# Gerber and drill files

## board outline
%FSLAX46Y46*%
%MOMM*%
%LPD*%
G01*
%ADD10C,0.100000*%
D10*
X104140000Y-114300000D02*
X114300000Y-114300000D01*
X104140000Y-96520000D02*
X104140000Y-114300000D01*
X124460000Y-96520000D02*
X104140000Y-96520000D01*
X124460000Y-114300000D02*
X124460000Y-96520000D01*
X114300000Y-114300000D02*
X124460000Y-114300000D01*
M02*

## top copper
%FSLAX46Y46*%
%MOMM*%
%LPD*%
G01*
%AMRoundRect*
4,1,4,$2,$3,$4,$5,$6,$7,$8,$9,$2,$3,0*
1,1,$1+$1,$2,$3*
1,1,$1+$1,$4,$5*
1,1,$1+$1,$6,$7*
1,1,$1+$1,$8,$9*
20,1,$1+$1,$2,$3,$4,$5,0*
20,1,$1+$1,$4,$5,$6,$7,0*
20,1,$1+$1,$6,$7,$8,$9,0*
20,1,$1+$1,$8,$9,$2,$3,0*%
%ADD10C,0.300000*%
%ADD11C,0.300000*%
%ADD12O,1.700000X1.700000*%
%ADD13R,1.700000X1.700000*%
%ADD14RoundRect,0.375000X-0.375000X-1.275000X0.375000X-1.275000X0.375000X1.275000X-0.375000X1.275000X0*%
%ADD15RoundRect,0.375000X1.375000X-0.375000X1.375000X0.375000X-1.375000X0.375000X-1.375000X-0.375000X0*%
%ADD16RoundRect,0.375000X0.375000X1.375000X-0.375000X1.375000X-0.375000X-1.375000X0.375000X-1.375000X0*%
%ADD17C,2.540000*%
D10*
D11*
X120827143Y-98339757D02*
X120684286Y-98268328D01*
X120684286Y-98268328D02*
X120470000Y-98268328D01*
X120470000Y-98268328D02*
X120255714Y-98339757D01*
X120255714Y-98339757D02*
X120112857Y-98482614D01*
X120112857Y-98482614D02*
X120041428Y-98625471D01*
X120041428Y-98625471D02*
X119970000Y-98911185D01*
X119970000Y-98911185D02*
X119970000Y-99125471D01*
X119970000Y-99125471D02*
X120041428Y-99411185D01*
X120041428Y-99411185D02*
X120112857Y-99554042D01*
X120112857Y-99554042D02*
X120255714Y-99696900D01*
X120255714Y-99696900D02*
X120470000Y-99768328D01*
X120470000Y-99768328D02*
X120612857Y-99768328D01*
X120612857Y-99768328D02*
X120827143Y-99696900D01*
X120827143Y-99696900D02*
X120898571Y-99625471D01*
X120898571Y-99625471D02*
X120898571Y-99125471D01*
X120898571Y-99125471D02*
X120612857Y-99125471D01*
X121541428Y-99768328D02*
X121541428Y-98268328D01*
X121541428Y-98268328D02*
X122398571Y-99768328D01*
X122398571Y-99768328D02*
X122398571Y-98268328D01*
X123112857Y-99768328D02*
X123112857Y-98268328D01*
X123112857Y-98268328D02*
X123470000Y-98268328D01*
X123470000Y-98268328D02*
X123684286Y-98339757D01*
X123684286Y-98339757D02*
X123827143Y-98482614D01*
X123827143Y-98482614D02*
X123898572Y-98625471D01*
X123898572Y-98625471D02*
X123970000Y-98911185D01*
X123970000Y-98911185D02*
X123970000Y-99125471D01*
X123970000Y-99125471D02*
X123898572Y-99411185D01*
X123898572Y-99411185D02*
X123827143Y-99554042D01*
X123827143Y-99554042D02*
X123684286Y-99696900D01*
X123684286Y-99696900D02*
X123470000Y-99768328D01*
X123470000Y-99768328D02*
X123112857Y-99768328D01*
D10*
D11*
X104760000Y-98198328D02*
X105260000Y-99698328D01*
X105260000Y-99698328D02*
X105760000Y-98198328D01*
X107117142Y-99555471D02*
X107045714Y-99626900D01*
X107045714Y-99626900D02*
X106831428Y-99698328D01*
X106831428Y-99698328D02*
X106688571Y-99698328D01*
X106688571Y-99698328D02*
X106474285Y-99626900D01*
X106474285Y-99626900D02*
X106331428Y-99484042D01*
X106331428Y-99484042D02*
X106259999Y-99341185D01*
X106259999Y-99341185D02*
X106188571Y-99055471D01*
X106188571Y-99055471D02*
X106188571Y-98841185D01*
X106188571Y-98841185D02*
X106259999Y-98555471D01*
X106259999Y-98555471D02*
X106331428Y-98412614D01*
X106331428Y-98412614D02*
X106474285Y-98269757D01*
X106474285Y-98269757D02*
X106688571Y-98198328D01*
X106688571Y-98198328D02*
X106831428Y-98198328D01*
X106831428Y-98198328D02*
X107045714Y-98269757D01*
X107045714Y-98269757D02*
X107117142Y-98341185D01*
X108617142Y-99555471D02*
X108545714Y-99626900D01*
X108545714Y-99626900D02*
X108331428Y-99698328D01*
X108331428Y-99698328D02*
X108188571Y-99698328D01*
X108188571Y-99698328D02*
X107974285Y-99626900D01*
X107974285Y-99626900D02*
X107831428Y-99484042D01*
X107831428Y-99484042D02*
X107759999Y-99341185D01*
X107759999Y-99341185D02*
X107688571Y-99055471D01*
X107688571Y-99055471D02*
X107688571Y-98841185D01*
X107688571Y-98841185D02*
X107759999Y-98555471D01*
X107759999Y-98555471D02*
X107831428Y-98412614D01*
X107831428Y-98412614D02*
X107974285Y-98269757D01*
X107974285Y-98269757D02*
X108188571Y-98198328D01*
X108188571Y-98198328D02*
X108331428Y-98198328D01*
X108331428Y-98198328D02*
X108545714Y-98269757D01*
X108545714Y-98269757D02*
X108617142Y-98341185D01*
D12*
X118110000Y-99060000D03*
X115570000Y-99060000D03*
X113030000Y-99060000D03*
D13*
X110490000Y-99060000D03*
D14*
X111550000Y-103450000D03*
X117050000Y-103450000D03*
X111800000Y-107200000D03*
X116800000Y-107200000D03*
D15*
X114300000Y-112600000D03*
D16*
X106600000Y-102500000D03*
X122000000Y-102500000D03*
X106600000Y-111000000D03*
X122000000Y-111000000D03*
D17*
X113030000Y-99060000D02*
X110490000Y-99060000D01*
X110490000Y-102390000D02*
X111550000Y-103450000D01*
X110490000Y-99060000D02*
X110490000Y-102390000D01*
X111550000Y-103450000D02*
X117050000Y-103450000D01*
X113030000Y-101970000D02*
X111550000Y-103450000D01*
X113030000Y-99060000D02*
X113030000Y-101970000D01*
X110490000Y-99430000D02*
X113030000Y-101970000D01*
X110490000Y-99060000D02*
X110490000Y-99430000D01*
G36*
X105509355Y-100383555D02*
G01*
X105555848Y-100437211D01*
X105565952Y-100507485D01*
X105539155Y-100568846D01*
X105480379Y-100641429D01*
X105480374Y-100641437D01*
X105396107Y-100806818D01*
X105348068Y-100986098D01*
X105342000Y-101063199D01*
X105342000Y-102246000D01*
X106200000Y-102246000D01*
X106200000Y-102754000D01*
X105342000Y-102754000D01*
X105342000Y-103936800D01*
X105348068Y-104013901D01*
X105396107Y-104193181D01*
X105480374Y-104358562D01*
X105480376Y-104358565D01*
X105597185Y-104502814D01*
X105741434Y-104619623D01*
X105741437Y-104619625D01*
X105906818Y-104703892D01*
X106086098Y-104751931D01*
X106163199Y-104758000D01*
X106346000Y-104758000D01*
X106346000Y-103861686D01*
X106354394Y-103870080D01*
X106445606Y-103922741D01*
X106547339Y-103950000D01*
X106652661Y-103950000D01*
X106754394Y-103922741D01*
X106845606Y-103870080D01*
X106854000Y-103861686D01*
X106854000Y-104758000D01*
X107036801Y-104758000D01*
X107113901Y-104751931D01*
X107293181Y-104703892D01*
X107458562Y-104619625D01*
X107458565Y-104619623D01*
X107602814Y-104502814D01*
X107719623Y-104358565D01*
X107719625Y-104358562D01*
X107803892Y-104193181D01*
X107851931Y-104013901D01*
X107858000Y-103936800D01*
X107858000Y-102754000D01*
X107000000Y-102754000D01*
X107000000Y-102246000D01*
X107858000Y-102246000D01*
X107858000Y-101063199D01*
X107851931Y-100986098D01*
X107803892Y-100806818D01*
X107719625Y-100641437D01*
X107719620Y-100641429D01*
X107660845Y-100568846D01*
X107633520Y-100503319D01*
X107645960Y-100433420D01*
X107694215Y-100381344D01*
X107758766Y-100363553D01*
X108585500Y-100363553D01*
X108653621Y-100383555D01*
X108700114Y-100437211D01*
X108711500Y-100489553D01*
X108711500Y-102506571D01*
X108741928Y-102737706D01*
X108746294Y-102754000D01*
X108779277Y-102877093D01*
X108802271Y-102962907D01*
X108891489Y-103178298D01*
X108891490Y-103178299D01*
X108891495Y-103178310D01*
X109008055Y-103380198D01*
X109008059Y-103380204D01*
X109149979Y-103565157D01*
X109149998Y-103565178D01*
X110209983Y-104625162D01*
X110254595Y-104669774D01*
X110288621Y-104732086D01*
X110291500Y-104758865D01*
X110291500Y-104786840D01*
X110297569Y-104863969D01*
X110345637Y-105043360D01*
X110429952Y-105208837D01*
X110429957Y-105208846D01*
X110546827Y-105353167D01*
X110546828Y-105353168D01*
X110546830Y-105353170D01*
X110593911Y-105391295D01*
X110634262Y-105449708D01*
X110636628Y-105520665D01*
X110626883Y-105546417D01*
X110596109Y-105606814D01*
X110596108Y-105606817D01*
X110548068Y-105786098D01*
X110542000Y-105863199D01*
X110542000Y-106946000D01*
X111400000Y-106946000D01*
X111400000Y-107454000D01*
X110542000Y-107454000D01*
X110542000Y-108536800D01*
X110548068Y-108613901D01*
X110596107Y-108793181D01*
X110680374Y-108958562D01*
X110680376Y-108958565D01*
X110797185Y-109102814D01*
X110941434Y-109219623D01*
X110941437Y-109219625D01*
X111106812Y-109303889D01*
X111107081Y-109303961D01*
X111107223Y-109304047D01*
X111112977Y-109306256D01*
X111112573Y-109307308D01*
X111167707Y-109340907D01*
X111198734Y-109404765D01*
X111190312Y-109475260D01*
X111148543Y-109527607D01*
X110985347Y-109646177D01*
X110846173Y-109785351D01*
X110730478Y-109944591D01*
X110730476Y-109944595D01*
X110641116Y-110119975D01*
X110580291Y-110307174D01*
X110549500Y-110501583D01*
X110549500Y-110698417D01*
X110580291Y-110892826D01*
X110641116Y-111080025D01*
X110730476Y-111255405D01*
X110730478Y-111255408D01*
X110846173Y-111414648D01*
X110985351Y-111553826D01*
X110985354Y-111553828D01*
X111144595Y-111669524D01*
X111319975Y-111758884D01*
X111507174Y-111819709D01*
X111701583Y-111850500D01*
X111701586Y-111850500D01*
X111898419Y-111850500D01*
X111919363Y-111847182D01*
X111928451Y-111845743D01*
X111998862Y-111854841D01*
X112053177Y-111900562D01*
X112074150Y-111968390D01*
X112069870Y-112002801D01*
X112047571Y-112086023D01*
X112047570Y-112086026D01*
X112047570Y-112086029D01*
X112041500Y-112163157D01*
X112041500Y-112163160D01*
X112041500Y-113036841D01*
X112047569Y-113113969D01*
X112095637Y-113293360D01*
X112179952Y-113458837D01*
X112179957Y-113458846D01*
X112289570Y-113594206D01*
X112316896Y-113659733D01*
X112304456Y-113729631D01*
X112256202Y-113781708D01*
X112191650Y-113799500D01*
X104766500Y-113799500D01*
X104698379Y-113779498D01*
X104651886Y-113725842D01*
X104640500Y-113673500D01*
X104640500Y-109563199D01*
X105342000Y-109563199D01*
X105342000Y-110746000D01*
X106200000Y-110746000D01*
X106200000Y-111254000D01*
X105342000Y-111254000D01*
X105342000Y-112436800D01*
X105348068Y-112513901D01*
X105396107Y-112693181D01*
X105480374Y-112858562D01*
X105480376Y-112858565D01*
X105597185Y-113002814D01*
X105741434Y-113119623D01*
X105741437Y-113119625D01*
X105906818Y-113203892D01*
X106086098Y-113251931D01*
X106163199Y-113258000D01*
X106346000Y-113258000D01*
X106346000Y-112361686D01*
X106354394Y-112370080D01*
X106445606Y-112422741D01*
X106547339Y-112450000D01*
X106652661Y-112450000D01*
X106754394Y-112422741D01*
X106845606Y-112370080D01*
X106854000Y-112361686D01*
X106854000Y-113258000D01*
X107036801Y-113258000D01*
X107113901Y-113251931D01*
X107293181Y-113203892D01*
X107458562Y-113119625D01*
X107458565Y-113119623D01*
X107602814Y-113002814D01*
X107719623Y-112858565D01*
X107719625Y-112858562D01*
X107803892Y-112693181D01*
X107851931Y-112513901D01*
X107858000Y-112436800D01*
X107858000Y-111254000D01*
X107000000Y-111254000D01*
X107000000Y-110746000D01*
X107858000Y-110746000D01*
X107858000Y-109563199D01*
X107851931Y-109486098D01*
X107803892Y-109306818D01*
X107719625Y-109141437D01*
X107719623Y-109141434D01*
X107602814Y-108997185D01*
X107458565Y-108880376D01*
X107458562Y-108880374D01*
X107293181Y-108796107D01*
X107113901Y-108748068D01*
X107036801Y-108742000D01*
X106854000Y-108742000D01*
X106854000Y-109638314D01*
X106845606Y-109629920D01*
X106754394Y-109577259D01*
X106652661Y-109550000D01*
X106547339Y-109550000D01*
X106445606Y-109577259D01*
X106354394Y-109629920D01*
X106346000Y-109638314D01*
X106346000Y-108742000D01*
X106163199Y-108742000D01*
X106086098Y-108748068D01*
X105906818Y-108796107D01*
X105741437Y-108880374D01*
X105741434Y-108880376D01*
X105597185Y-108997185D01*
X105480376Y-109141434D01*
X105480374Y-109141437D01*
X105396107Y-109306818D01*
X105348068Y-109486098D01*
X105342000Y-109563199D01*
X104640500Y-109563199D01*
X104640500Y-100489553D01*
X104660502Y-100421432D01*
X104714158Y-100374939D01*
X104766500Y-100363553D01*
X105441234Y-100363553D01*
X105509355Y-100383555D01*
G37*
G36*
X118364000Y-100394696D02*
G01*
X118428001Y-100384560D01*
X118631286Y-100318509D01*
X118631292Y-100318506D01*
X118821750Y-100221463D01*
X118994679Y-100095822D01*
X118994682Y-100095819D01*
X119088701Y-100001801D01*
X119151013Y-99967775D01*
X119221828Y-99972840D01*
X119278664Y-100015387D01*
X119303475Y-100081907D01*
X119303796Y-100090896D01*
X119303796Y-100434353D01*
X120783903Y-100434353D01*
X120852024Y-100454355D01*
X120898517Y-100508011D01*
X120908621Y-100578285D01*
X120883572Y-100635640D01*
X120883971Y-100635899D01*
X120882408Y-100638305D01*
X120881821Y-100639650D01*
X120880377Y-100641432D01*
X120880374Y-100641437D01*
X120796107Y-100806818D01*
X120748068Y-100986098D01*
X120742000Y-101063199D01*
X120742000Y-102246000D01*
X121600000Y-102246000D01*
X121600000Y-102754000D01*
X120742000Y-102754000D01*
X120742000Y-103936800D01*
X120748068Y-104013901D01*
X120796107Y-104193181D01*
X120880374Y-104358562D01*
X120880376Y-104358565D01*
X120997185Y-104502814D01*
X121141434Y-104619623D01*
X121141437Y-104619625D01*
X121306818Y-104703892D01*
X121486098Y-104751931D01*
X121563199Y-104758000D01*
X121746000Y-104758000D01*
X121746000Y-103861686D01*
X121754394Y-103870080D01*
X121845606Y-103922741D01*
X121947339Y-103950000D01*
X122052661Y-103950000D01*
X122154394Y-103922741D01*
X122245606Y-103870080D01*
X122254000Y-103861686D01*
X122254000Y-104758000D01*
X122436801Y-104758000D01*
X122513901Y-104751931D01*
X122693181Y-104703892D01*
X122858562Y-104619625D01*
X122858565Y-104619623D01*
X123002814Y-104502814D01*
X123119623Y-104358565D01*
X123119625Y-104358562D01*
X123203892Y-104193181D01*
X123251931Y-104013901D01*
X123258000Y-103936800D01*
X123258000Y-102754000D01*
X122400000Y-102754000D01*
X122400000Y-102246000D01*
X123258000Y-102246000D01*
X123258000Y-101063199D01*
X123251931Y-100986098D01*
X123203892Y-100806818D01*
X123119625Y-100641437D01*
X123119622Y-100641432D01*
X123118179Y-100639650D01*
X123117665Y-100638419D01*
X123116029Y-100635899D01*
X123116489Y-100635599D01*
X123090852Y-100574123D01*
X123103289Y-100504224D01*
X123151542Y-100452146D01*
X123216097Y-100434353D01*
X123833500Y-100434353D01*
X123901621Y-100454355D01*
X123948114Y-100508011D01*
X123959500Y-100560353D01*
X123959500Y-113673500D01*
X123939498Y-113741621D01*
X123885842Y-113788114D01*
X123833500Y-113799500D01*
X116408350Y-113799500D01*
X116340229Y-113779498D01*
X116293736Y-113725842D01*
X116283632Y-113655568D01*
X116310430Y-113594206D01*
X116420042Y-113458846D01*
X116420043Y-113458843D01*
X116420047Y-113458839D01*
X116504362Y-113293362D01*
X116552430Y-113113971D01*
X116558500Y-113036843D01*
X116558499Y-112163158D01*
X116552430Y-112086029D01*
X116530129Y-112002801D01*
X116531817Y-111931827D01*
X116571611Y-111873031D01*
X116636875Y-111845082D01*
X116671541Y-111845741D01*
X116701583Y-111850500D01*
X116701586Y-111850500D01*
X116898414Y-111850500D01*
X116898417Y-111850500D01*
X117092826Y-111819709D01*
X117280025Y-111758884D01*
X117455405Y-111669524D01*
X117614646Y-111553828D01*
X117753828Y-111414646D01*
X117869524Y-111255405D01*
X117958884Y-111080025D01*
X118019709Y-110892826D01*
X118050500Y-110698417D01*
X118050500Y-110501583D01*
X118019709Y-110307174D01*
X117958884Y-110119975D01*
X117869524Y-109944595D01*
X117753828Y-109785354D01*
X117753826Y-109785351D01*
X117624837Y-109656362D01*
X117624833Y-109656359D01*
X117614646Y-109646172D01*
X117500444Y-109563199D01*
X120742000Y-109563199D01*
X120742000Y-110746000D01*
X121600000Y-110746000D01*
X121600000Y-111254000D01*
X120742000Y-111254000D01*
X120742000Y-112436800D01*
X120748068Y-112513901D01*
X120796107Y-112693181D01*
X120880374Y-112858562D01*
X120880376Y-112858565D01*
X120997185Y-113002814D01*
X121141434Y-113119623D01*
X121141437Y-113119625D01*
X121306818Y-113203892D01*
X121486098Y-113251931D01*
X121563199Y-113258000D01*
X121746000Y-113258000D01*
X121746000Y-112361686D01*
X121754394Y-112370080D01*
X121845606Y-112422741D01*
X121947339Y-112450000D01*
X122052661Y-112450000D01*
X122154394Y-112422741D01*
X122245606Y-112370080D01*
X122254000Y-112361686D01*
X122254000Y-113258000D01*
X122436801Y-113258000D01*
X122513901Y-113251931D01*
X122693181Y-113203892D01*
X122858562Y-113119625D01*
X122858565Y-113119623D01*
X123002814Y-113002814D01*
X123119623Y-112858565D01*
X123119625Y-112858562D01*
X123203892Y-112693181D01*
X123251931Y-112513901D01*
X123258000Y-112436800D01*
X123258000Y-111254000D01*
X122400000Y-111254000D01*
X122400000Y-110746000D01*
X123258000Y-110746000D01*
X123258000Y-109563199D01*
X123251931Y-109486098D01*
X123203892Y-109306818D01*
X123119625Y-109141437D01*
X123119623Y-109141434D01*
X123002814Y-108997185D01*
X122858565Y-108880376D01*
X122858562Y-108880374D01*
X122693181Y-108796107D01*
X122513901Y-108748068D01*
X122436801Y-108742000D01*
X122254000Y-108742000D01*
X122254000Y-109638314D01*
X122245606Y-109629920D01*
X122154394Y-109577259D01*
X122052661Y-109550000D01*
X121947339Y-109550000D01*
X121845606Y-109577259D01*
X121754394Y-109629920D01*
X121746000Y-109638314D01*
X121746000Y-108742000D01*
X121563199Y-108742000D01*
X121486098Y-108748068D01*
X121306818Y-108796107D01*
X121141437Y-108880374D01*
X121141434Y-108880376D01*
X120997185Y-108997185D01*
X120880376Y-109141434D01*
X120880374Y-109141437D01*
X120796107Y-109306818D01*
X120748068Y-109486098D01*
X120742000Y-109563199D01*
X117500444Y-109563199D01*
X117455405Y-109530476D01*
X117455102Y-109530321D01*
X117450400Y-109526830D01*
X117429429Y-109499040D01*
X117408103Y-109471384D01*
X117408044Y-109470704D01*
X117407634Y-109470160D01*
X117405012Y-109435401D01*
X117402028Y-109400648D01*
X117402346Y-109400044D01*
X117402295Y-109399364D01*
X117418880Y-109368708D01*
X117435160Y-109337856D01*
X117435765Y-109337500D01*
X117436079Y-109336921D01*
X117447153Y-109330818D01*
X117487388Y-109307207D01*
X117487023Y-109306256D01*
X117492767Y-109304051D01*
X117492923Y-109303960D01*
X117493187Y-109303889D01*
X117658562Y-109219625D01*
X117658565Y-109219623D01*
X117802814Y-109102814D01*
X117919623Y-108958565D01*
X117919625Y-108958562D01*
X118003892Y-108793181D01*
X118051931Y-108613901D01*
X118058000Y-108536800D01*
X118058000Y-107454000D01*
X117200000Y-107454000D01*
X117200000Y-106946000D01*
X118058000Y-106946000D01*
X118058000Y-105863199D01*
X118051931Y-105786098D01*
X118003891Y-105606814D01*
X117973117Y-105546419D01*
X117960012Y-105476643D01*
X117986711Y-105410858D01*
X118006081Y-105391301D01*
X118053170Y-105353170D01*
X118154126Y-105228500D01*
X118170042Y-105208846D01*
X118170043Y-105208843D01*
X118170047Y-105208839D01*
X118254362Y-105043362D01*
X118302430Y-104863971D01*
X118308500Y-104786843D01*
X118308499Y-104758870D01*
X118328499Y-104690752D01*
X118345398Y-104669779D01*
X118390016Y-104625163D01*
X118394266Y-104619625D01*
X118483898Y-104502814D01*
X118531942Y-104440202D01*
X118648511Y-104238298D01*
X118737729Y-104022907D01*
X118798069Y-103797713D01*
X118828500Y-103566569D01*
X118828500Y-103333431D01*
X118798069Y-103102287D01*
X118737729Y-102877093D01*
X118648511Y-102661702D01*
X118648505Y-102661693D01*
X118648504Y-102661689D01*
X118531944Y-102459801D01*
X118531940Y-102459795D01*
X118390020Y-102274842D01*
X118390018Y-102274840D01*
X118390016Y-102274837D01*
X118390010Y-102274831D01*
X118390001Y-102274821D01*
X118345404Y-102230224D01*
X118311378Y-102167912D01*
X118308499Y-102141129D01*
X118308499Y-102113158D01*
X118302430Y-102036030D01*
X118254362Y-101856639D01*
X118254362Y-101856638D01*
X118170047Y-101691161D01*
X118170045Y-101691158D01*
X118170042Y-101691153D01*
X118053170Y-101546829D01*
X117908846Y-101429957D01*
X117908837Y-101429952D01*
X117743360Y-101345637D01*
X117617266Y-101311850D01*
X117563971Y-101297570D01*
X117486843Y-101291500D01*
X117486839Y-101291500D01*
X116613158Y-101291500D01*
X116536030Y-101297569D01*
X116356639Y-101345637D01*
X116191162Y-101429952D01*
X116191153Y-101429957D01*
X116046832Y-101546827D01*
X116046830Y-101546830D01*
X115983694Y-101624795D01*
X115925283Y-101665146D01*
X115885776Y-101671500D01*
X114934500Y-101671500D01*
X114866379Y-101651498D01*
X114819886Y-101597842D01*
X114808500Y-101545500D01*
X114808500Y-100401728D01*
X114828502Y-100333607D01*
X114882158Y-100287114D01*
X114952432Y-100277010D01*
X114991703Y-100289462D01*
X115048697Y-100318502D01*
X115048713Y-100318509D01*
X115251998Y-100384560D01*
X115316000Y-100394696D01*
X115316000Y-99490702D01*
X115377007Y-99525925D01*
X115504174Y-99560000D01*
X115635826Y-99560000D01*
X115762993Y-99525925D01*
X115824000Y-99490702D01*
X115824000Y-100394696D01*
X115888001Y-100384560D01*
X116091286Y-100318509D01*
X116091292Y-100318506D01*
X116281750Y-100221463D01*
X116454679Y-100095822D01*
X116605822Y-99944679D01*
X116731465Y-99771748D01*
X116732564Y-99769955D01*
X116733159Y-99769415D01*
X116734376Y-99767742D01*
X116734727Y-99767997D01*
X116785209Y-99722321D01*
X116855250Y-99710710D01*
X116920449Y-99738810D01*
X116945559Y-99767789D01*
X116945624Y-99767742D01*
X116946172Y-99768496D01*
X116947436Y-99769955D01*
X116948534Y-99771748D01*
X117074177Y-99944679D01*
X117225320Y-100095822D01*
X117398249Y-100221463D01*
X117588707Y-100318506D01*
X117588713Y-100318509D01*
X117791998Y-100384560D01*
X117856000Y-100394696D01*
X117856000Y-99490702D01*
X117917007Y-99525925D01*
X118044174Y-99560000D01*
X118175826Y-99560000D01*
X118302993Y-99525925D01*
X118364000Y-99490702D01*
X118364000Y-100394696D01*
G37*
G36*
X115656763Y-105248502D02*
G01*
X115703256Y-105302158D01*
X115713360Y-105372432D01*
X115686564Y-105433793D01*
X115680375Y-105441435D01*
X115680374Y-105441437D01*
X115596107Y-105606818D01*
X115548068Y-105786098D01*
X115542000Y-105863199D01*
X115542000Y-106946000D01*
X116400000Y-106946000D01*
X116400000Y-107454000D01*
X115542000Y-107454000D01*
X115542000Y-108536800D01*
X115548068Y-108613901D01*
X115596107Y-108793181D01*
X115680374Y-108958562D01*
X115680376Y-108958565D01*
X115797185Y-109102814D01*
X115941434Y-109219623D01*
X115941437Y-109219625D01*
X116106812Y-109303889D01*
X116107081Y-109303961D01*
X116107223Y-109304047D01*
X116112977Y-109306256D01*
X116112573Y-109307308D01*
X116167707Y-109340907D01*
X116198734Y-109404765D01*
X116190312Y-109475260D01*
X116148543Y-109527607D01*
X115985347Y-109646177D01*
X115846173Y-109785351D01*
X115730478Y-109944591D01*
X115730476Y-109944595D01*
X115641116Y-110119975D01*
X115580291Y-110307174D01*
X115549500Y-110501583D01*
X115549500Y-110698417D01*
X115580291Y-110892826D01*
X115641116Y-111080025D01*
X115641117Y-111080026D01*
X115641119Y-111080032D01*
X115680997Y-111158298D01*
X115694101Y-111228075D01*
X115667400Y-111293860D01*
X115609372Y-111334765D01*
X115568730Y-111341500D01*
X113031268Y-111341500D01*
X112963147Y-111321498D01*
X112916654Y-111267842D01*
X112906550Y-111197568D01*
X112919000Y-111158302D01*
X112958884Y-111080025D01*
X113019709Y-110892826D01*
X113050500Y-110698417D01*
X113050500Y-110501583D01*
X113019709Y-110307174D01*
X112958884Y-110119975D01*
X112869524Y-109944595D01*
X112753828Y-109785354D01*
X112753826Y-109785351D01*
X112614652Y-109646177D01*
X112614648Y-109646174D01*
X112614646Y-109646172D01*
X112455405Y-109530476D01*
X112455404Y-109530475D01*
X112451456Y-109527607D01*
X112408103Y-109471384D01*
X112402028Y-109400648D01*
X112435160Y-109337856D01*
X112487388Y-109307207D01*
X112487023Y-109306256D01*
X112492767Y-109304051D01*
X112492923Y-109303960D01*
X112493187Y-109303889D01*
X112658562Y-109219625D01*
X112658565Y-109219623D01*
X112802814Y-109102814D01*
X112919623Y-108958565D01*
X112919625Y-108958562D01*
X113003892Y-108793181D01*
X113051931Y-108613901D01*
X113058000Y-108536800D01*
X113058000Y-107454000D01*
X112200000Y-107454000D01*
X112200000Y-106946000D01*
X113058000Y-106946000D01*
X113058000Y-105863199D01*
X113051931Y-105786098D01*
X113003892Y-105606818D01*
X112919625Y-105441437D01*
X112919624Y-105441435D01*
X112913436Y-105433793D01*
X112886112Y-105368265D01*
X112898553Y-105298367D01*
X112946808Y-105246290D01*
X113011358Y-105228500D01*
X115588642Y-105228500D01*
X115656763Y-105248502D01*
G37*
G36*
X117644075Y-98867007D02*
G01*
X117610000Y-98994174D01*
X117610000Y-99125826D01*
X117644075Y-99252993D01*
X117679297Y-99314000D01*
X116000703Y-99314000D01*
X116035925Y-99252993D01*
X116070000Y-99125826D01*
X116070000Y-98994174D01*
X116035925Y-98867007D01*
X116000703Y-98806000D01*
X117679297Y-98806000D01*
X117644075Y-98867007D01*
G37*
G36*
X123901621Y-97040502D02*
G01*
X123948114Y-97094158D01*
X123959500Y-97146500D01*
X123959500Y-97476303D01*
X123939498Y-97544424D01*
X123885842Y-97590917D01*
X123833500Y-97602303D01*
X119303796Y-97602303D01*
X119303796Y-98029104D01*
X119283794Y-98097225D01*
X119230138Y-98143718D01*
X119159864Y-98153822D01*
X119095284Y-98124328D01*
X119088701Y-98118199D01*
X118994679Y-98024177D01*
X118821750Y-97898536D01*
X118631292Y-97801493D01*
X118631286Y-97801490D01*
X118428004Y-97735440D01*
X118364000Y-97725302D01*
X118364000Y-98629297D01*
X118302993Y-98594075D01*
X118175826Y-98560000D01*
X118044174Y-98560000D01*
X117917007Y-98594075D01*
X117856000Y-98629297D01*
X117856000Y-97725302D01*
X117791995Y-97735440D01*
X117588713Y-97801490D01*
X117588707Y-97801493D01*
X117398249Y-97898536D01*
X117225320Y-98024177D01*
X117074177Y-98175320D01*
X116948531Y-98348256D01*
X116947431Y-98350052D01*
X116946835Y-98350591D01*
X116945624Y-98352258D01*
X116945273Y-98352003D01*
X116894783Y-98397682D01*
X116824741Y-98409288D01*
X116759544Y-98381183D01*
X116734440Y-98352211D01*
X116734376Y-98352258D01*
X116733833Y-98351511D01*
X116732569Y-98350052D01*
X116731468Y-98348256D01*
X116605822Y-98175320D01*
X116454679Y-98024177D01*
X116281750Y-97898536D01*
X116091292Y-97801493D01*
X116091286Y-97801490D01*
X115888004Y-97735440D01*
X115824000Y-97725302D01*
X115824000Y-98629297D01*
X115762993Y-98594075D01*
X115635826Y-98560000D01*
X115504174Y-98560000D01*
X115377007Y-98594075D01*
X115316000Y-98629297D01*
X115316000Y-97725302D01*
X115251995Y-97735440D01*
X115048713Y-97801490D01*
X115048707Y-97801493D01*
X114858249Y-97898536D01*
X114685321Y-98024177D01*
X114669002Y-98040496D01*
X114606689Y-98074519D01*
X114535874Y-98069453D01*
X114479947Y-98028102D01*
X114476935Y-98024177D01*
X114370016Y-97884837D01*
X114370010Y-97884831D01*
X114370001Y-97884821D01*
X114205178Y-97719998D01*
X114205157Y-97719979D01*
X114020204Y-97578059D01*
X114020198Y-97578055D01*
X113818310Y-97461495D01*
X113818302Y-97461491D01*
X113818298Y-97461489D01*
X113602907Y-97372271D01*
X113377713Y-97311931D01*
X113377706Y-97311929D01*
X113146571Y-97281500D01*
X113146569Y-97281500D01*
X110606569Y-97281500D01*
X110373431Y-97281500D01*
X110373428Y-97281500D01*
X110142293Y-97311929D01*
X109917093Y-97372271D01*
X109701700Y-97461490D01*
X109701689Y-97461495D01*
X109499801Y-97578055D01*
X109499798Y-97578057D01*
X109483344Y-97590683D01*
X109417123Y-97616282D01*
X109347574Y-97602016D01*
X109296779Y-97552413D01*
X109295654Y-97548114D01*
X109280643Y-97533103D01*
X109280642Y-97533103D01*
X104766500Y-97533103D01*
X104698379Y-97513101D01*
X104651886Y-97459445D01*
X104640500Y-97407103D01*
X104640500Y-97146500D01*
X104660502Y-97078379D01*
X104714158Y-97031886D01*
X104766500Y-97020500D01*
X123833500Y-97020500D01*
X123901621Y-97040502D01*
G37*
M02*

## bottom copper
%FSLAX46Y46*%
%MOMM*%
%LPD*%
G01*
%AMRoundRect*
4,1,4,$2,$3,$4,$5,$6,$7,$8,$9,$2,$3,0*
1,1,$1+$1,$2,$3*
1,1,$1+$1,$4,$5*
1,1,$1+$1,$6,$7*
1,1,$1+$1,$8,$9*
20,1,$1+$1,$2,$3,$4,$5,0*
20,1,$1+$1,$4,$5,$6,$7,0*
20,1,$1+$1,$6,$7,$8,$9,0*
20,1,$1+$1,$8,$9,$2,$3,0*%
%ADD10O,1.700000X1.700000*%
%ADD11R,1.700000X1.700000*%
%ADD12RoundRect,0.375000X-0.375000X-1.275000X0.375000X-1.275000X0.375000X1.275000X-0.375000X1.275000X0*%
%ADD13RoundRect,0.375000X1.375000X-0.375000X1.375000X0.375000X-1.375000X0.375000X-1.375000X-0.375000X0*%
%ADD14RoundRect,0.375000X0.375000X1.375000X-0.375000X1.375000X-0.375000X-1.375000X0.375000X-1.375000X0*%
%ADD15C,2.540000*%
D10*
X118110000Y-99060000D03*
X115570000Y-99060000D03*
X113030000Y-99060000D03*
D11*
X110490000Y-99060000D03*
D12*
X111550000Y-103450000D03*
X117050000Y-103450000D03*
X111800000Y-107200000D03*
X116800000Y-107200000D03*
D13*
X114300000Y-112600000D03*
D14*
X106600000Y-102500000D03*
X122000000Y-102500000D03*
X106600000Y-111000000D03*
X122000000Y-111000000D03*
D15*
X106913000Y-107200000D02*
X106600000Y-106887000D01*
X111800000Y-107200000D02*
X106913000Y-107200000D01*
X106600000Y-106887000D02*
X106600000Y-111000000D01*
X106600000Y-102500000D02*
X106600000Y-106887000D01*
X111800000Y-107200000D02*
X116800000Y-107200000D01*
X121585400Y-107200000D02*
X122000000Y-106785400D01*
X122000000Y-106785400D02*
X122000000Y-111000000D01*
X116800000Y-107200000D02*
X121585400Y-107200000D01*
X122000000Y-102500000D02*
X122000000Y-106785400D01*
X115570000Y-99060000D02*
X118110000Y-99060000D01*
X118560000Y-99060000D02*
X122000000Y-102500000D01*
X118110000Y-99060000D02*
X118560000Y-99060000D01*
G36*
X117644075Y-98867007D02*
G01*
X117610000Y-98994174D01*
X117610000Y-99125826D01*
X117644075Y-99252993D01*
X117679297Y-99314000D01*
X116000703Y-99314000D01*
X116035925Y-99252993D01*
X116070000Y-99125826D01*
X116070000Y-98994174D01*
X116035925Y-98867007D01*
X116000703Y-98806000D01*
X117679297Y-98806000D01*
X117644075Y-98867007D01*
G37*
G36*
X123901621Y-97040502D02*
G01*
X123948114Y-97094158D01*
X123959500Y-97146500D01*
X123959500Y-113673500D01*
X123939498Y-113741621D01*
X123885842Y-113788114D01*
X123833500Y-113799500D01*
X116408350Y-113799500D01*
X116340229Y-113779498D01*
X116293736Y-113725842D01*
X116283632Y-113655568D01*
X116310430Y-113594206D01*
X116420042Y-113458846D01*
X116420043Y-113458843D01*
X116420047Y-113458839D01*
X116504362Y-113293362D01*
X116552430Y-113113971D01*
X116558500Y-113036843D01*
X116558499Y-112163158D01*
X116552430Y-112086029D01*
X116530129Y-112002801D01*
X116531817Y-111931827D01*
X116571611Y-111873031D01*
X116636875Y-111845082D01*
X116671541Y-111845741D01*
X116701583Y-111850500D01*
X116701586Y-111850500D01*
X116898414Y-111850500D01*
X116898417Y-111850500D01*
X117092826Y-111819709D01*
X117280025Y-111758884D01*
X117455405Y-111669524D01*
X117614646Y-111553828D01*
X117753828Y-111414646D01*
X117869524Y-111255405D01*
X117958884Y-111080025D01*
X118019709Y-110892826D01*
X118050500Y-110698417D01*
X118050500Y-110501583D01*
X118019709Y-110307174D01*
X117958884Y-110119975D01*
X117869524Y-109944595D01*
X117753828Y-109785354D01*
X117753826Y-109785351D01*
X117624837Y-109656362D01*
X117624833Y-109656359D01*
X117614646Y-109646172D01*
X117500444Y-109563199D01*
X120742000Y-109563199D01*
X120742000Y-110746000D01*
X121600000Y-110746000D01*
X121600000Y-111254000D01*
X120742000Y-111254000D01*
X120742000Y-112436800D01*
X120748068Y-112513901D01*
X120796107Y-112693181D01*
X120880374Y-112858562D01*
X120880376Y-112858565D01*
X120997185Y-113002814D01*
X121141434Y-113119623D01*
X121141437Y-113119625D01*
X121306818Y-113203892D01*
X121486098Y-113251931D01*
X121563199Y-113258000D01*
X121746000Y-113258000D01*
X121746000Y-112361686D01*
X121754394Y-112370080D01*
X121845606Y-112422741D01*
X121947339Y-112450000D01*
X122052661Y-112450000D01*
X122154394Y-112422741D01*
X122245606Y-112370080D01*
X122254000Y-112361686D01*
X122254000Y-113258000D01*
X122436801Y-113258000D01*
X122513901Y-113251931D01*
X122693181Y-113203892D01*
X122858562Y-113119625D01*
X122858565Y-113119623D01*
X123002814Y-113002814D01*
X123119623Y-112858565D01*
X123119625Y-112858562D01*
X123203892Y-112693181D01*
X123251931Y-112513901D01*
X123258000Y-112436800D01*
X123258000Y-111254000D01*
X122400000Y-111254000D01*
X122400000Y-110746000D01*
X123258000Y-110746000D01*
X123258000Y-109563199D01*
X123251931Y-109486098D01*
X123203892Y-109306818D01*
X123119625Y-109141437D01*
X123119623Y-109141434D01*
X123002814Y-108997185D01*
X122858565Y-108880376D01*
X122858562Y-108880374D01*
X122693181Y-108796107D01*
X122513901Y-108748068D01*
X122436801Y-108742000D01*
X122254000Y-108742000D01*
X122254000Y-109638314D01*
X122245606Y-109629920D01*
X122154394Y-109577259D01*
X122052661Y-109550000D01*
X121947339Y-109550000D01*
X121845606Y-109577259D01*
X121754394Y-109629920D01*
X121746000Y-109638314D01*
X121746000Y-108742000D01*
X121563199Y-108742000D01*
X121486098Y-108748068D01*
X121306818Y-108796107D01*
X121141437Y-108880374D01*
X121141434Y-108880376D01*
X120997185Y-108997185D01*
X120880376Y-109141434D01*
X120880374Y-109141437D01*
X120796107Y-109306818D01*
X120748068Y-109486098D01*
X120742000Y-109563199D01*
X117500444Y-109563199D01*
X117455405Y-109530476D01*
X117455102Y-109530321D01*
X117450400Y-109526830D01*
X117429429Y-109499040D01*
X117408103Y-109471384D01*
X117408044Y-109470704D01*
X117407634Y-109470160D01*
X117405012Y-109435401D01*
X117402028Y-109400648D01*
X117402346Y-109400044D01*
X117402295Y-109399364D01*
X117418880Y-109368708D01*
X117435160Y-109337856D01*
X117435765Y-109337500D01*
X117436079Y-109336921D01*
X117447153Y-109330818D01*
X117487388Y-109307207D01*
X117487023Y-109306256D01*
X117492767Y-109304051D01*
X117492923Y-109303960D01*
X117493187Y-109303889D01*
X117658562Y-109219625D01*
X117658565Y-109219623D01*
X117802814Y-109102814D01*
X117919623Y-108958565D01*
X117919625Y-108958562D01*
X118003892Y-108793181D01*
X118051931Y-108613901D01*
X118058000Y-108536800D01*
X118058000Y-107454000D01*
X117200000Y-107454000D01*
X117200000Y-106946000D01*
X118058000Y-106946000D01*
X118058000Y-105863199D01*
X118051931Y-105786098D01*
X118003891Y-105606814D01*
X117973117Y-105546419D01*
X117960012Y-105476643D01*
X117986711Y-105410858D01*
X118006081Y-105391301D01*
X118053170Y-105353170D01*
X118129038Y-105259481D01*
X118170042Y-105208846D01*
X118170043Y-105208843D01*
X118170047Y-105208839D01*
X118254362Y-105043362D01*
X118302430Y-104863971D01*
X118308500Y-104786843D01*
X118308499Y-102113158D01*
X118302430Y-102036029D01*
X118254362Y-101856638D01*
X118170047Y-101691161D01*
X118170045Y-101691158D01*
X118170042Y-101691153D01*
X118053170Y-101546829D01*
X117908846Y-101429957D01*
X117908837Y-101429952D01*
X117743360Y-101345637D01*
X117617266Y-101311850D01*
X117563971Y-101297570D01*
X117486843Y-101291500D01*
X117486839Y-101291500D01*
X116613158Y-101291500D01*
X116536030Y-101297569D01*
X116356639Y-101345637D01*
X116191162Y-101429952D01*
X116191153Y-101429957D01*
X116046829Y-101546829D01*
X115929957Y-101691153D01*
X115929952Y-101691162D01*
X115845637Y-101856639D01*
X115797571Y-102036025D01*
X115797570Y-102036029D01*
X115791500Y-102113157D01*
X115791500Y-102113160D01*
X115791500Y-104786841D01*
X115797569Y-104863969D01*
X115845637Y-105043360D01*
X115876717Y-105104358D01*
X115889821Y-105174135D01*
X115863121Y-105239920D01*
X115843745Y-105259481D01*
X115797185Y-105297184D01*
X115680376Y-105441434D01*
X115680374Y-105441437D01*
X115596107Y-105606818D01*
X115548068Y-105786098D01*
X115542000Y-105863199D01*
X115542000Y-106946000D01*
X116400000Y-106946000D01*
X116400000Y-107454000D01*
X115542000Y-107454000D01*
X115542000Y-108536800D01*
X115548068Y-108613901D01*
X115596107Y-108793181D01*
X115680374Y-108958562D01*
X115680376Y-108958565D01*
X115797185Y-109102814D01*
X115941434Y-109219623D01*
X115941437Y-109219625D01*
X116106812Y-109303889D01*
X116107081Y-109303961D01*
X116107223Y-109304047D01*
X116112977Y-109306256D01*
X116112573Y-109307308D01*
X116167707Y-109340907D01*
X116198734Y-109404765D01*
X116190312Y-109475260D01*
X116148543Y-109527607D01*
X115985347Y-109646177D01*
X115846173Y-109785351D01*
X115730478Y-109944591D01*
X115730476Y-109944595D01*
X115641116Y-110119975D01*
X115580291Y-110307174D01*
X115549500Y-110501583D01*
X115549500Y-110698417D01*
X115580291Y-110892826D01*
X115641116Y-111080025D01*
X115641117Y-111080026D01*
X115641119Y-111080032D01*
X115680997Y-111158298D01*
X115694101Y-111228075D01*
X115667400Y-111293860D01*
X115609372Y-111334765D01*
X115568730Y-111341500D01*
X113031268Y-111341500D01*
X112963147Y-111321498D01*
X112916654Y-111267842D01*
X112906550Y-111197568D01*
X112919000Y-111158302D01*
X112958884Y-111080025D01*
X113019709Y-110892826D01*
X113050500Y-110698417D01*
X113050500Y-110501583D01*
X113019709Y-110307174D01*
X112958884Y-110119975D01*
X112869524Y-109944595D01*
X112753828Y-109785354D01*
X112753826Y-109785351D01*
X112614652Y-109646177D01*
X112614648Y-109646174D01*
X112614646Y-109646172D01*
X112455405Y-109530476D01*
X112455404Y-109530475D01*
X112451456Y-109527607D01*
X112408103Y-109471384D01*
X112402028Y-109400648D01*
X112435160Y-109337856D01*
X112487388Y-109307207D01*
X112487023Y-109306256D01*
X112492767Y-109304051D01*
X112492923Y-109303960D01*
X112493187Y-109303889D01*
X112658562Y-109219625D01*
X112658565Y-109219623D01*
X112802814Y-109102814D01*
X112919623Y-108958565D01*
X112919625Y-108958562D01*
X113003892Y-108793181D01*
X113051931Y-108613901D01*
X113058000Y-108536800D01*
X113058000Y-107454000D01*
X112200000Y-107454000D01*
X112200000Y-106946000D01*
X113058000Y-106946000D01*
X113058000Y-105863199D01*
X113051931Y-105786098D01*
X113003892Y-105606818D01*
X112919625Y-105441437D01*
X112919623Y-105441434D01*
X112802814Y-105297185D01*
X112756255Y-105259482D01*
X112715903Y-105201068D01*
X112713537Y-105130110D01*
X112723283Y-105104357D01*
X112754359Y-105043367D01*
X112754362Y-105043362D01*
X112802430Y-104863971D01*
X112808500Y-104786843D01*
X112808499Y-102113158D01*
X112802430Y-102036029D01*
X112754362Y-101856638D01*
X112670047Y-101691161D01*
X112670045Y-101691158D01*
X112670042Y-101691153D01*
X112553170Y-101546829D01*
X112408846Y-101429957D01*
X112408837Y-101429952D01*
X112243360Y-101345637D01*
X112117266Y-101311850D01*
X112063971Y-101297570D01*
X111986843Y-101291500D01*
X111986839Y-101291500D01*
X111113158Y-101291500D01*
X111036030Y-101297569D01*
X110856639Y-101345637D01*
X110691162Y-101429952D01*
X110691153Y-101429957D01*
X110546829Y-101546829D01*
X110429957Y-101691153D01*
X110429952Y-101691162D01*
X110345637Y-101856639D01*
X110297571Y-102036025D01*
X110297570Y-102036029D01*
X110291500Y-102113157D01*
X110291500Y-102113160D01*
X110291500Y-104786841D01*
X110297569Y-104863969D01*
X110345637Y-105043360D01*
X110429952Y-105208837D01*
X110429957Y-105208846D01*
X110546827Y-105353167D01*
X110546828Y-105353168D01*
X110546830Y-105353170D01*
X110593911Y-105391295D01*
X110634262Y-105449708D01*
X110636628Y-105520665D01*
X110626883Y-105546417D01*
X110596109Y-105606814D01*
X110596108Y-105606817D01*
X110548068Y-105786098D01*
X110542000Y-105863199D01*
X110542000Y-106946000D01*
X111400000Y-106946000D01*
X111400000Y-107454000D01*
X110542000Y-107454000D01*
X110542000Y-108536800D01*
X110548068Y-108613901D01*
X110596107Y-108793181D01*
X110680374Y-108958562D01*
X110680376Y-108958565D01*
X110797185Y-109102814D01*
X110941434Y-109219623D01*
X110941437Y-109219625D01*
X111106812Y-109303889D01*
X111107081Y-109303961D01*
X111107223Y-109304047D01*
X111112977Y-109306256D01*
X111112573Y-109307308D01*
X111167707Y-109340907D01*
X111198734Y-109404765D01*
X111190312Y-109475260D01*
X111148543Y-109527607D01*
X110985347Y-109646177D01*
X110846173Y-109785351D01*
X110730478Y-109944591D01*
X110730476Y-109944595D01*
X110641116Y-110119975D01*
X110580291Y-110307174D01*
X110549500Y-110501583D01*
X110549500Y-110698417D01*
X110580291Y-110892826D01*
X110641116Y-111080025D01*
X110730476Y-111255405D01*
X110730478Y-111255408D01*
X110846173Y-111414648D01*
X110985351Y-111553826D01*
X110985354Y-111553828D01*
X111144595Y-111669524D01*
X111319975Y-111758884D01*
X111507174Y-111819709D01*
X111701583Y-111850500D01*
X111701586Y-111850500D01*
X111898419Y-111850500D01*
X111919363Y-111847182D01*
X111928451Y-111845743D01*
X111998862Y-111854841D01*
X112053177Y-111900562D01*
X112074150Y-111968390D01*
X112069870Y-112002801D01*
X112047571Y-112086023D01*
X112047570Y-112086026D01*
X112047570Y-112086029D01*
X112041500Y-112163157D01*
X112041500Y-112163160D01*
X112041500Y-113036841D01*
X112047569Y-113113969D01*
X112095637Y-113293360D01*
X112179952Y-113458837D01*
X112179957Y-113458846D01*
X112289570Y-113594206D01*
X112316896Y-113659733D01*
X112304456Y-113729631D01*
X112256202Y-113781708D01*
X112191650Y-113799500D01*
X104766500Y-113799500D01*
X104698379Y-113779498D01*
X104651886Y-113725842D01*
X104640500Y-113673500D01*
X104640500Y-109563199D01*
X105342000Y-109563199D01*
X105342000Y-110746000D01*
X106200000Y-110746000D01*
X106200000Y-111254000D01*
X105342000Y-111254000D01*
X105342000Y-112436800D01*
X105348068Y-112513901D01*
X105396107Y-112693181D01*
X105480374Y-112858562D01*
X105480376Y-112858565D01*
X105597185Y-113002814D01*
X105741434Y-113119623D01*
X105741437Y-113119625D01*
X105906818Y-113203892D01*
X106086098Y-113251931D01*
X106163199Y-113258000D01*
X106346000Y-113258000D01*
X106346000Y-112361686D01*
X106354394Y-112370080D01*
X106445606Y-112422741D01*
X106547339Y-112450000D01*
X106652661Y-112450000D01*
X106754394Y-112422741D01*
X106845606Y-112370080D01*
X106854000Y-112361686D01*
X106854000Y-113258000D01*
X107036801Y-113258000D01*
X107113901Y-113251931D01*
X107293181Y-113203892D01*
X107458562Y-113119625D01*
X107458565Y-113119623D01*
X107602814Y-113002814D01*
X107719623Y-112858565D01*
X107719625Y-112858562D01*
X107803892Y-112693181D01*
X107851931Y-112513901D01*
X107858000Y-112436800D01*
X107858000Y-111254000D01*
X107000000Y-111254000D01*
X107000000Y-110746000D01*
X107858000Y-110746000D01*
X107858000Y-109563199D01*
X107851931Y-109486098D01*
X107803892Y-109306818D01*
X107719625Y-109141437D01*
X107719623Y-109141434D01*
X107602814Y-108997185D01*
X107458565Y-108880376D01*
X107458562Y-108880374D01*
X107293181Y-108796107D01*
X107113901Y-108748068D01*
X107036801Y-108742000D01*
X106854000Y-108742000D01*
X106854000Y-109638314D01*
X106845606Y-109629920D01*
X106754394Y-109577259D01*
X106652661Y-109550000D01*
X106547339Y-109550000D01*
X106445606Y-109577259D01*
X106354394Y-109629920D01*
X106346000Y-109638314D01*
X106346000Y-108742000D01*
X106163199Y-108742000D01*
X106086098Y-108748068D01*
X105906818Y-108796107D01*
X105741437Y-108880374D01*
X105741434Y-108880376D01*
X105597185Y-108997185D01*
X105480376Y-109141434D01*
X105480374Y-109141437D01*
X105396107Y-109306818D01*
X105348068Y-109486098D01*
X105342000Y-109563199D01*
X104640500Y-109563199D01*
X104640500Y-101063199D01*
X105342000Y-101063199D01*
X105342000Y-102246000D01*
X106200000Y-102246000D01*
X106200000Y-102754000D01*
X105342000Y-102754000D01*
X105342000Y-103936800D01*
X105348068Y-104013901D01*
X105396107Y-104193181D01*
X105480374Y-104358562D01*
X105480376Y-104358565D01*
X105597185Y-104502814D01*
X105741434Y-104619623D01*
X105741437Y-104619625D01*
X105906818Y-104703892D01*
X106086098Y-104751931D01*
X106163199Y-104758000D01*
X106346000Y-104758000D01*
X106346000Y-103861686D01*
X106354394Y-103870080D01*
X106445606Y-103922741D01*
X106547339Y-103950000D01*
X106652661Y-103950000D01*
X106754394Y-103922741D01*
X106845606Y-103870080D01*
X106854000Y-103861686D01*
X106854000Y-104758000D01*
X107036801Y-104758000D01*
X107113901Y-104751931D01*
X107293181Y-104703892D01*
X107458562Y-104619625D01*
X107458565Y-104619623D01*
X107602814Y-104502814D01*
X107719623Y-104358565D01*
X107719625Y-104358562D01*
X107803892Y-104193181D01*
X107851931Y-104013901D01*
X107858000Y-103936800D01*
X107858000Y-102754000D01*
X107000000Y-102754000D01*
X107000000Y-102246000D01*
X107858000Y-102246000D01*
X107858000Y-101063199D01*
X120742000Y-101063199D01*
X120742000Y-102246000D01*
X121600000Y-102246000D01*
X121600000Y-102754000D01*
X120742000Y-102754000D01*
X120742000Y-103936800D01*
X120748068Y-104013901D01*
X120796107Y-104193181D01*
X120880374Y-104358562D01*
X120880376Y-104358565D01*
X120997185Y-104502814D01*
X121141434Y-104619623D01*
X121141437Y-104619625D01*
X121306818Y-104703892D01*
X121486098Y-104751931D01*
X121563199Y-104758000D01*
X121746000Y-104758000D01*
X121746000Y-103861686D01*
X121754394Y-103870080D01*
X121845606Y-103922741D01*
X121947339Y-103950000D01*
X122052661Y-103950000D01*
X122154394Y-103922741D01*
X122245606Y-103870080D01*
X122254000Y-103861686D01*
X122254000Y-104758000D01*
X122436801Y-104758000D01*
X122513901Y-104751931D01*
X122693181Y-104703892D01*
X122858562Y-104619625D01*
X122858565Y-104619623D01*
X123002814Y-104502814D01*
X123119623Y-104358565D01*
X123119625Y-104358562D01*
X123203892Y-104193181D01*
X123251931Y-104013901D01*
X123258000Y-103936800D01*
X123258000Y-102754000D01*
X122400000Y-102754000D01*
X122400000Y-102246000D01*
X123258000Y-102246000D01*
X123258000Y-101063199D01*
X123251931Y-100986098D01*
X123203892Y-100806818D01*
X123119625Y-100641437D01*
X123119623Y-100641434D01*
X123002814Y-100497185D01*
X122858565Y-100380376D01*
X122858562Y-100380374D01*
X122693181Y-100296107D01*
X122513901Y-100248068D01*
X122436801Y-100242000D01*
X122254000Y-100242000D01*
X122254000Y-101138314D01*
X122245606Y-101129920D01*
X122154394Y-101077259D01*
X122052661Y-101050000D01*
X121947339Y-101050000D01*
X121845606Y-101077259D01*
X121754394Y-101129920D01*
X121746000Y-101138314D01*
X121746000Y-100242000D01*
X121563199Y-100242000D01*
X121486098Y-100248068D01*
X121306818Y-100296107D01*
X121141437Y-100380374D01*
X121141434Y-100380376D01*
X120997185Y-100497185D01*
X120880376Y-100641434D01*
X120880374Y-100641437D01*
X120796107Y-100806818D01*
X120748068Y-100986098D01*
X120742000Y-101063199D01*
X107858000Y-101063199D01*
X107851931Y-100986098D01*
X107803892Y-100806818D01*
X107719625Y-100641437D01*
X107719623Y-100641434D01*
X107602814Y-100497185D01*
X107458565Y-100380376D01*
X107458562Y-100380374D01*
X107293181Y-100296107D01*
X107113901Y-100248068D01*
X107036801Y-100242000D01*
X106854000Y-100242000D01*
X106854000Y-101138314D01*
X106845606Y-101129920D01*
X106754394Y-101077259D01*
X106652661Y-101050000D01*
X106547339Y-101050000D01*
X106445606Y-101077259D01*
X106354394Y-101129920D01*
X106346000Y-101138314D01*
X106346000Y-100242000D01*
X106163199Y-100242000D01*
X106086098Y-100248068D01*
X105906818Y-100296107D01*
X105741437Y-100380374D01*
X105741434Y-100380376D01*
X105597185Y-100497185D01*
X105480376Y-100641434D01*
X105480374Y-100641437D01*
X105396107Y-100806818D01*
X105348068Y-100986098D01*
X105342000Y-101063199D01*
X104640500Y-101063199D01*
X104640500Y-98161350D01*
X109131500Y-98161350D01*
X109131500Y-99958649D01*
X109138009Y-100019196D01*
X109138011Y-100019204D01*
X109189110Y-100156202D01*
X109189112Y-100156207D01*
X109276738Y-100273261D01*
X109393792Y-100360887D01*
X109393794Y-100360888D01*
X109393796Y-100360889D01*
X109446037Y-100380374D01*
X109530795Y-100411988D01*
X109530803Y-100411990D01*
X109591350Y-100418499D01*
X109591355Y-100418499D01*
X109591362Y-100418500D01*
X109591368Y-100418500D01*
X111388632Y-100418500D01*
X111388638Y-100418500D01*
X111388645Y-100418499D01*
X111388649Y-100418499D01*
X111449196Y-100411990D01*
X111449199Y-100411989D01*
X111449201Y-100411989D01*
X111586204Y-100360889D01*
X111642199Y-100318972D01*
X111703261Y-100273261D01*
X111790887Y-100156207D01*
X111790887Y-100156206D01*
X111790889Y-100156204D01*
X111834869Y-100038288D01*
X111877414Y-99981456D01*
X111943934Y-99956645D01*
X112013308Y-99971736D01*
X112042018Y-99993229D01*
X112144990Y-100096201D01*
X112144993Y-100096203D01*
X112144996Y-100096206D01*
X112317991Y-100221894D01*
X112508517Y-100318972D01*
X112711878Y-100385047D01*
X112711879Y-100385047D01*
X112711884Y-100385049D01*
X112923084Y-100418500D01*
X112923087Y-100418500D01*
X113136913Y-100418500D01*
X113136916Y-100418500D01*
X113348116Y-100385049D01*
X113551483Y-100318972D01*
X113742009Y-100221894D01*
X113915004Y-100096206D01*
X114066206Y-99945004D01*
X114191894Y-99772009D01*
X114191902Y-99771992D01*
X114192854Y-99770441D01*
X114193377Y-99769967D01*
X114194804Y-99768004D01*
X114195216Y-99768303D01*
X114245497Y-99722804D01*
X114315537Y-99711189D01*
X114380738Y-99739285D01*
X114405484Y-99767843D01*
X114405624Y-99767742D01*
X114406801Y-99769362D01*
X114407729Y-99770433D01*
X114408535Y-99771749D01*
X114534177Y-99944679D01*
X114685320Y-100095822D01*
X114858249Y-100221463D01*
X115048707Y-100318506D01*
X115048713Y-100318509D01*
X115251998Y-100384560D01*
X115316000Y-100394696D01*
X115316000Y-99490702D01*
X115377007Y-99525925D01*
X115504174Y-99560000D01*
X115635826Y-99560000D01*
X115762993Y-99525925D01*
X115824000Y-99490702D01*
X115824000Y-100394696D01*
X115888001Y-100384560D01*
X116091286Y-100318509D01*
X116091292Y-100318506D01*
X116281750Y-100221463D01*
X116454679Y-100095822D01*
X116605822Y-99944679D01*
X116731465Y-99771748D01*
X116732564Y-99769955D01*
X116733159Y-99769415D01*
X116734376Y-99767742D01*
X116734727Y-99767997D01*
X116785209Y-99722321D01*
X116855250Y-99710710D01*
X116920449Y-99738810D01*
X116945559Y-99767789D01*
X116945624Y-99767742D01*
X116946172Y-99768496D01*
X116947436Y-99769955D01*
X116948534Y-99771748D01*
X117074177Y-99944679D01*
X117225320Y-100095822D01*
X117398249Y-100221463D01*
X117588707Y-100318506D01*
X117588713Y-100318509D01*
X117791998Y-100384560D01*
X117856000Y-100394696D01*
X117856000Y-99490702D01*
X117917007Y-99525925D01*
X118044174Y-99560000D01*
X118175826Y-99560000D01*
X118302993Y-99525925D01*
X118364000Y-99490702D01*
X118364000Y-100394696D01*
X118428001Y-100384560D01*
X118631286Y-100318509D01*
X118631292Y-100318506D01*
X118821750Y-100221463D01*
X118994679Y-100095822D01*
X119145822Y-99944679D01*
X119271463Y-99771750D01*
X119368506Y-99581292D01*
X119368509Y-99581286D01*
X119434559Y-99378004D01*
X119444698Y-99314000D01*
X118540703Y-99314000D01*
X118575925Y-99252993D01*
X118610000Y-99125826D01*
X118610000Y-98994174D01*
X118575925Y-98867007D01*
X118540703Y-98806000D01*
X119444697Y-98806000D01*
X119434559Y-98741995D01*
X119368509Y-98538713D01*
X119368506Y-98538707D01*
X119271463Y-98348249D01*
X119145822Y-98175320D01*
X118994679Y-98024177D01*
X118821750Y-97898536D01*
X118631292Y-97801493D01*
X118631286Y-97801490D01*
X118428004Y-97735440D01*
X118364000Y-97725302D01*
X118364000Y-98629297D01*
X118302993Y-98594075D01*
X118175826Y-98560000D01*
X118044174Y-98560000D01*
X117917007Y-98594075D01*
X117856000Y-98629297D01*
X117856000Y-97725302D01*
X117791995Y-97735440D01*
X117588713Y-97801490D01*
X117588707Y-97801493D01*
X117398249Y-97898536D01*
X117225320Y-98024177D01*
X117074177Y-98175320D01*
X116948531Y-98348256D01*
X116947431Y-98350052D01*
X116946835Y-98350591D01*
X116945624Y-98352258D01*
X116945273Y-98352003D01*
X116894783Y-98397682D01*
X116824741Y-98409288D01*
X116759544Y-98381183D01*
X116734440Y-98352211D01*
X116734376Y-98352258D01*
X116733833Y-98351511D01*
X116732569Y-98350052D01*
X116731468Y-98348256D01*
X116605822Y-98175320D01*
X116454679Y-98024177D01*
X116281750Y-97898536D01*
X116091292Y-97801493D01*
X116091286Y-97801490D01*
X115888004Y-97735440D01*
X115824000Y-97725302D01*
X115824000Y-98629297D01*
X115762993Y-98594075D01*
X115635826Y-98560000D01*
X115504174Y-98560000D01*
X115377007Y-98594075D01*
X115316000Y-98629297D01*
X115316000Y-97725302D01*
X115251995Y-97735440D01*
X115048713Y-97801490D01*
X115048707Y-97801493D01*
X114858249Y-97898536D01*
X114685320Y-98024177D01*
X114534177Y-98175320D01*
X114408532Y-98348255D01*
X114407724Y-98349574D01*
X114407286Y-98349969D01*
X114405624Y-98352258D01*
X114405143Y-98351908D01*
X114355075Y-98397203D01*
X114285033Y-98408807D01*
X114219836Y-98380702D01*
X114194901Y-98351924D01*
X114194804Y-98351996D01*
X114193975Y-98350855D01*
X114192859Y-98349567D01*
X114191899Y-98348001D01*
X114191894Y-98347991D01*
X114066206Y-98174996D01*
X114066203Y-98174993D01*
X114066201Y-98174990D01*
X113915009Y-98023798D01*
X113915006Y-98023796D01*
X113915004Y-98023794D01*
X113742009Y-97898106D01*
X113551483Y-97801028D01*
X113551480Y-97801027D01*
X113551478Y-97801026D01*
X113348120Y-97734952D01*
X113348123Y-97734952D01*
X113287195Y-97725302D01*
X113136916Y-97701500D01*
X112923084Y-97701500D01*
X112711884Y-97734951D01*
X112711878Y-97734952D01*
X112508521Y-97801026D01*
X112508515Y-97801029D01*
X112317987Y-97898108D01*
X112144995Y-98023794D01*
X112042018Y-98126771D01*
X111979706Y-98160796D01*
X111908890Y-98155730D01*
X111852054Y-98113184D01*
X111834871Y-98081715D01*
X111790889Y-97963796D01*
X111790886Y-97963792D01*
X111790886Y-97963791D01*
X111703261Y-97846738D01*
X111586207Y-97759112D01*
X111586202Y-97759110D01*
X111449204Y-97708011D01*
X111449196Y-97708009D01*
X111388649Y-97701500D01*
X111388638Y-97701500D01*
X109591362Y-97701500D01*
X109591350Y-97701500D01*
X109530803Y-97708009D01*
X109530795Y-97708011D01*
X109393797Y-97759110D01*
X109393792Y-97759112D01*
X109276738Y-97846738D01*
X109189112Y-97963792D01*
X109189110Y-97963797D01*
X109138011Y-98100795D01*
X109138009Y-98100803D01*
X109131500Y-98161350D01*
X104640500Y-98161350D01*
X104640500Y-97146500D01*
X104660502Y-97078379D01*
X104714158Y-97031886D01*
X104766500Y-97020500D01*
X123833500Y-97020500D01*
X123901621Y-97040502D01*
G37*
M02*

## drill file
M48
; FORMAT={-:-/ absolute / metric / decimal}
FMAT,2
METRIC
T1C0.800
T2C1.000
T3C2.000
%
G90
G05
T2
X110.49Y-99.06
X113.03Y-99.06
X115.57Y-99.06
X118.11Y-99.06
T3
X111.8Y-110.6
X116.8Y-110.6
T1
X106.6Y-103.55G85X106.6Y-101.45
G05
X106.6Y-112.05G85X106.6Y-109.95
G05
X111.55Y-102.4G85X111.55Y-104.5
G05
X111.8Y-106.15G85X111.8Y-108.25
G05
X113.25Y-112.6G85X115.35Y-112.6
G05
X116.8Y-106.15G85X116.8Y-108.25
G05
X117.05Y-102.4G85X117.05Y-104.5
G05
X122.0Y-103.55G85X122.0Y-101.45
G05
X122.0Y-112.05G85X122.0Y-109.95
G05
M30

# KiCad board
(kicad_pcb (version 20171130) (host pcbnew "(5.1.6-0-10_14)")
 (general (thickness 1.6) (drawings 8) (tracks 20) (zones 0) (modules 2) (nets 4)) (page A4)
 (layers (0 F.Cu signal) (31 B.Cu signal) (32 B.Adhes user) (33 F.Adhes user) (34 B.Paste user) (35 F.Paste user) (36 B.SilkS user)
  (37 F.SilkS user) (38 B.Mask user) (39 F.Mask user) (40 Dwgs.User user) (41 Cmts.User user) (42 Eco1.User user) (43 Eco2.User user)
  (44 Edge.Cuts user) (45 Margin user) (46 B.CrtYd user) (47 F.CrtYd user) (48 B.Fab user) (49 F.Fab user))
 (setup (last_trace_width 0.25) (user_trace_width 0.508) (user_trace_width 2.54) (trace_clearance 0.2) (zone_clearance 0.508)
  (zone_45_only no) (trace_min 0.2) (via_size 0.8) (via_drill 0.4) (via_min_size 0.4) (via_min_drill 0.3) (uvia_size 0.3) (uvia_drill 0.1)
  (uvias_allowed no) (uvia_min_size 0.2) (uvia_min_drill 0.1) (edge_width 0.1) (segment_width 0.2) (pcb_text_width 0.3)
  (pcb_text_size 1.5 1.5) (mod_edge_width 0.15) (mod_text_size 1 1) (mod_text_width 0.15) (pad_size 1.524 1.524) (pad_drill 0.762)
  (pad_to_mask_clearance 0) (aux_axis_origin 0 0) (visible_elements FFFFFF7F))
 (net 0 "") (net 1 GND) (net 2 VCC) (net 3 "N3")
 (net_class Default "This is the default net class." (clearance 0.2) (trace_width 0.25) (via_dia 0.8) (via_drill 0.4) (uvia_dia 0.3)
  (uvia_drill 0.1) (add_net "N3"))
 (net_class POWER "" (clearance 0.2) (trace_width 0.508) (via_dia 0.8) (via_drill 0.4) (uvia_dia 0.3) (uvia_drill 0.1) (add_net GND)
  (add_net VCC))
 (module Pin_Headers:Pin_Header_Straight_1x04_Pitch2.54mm (layer F.Cu) (at 110.49 99.06 90)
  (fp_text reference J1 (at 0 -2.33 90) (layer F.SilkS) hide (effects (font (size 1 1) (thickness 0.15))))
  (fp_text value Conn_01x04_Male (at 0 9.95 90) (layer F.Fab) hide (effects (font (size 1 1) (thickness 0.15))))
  (pad 4 thru_hole oval (at 0 7.62 90) (size 1.7 1.7) (drill 1) (layers *.Cu *.Mask) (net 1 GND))
  (pad 3 thru_hole oval (at 0 5.08 90) (size 1.7 1.7) (drill 1) (layers *.Cu *.Mask) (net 1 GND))
  (pad 2 thru_hole oval (at 0 2.54 90) (size 1.7 1.7) (drill 1) (layers *.Cu *.Mask) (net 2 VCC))
  (pad 1 thru_hole rect (at 0 0 90) (size 1.7 1.7) (drill 1) (layers *.Cu *.Mask) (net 2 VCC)))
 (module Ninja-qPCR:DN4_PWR (layer F.Cu) (at 114.3 114.3)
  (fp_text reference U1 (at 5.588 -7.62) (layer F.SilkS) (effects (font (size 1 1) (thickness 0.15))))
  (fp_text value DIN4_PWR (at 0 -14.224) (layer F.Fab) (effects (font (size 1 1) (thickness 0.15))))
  (pad 1 thru_hole roundrect (at -2.75 -10.85) (size 1.5 3.3) (drill oval 0.8 2.9) (layers *.Cu *.Mask) (roundrect_rratio 0.25) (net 2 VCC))
  (pad 2 thru_hole roundrect (at 2.75 -10.85) (size 1.5 3.3) (drill oval 0.8 2.9) (layers *.Cu *.Mask) (roundrect_rratio 0.25) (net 2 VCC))
  (pad 3 thru_hole roundrect (at -2.5 -7.1) (size 1.5 3.3) (drill oval 0.8 2.9) (layers *.Cu *.Mask) (roundrect_rratio 0.25) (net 1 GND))
  (pad 4 thru_hole roundrect (at 2.5 -7.1) (size 1.5 3.3) (drill oval 0.8 2.9) (layers *.Cu *.Mask) (roundrect_rratio 0.25) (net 1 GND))
  (pad 5 thru_hole roundrect (at 0 -1.7 90) (size 1.5 3.5) (drill oval 0.8 2.9) (layers *.Cu *.Mask) (roundrect_rratio 0.25) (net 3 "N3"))
  (pad 6 thru_hole roundrect (at -7.7 -11.8 180) (size 1.5 3.5) (drill oval 0.8 2.9) (layers *.Cu *.Mask) (roundrect_rratio 0.25)
   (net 1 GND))
  (pad 8 thru_hole roundrect (at 7.7 -11.8 180) (size 1.5 3.5) (drill oval 0.8 2.9) (layers *.Cu *.Mask) (roundrect_rratio 0.25) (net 1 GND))
  (pad 7 thru_hole roundrect (at -7.7 -3.3 180) (size 1.5 3.5) (drill oval 0.8 2.9) (layers *.Cu *.Mask) (roundrect_rratio 0.25) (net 1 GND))
  (pad 9 thru_hole roundrect (at 7.7 -3.3 180) (size 1.5 3.5) (drill oval 0.8 2.9) (layers *.Cu *.Mask) (roundrect_rratio 0.25) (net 1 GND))
  (pad "" np_thru_hole circle (at -2.5 -3.7) (size 2 2) (drill 2) (layers *.Cu *.Mask))
  (pad "" np_thru_hole circle (at 2.5 -3.7) (size 2 2) (drill 2) (layers *.Cu *.Mask)))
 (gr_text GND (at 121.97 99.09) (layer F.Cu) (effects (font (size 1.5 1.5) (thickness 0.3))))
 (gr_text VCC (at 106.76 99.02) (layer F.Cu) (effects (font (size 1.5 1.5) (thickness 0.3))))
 (gr_line (start 104.14 114.3) (end 114.3 114.3) (layer Edge.Cuts) (width 0.1))
 (gr_line (start 104.14 96.52) (end 104.14 114.3) (layer Edge.Cuts) (width 0.1))
 (gr_line (start 124.46 96.52) (end 104.14 96.52) (layer Edge.Cuts) (width 0.1))
 (gr_line (start 124.46 114.3) (end 124.46 96.52) (layer Edge.Cuts) (width 0.1))
 (gr_line (start 114.3 114.3) (end 124.46 114.3) (layer Edge.Cuts) (width 0.1))
 (segment (start 106.913 107.2) (end 106.6 106.887) (width 2.54) (layer B.Cu) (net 1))
 (segment (start 111.8 107.2) (end 106.913 107.2) (width 2.54) (layer B.Cu) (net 1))
 (segment (start 106.6 106.887) (end 106.6 111) (width 2.54) (layer B.Cu) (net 1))
 (segment (start 106.6 102.5) (end 106.6 106.887) (width 2.54) (layer B.Cu) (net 1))
 (segment (start 111.8 107.2) (end 116.8 107.2) (width 2.54) (layer B.Cu) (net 1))
 (segment (start 121.5854 107.2) (end 122 106.7854) (width 2.54) (layer B.Cu) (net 1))
 (segment (start 122 106.7854) (end 122 111) (width 2.54) (layer B.Cu) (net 1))
 (segment (start 116.8 107.2) (end 121.5854 107.2) (width 2.54) (layer B.Cu) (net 1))
 (segment (start 122 102.5) (end 122 106.7854) (width 2.54) (layer B.Cu) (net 1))
 (segment (start 115.57 99.06) (end 118.11 99.06) (width 2.54) (layer B.Cu) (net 1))
 (segment (start 118.56 99.06) (end 122 102.5) (width 2.54) (layer B.Cu) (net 1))
 (segment (start 118.11 99.06) (end 118.56 99.06) (width 2.54) (layer B.Cu) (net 1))
 (segment (start 113.03 99.06) (end 110.49 99.06) (width 2.54) (layer F.Cu) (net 2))
 (segment (start 110.49 102.39) (end 111.55 103.45) (width 2.54) (layer F.Cu) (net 2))
 (segment (start 110.49 99.06) (end 110.49 102.39) (width 2.54) (layer F.Cu) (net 2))
 (segment (start 111.55 103.45) (end 117.05 103.45) (width 2.54) (layer F.Cu) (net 2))
 (segment (start 113.03 101.97) (end 111.55 103.45) (width 2.54) (layer F.Cu) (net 2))
 (segment (start 113.03 99.06) (end 113.03 101.97) (width 2.54) (layer F.Cu) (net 2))
 (segment (start 110.49 99.43) (end 113.03 101.97) (width 2.54) (layer F.Cu) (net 2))
 (segment (start 110.49 99.06) (end 110.49 99.43) (width 2.54) (layer F.Cu) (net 2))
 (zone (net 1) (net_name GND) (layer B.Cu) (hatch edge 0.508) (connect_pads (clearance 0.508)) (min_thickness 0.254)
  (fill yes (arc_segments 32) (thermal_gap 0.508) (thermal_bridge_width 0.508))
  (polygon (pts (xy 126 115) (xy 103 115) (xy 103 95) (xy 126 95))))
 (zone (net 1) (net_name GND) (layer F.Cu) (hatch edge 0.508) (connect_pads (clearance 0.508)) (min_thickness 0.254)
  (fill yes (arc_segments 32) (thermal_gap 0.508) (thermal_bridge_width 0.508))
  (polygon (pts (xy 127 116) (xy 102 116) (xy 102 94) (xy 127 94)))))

